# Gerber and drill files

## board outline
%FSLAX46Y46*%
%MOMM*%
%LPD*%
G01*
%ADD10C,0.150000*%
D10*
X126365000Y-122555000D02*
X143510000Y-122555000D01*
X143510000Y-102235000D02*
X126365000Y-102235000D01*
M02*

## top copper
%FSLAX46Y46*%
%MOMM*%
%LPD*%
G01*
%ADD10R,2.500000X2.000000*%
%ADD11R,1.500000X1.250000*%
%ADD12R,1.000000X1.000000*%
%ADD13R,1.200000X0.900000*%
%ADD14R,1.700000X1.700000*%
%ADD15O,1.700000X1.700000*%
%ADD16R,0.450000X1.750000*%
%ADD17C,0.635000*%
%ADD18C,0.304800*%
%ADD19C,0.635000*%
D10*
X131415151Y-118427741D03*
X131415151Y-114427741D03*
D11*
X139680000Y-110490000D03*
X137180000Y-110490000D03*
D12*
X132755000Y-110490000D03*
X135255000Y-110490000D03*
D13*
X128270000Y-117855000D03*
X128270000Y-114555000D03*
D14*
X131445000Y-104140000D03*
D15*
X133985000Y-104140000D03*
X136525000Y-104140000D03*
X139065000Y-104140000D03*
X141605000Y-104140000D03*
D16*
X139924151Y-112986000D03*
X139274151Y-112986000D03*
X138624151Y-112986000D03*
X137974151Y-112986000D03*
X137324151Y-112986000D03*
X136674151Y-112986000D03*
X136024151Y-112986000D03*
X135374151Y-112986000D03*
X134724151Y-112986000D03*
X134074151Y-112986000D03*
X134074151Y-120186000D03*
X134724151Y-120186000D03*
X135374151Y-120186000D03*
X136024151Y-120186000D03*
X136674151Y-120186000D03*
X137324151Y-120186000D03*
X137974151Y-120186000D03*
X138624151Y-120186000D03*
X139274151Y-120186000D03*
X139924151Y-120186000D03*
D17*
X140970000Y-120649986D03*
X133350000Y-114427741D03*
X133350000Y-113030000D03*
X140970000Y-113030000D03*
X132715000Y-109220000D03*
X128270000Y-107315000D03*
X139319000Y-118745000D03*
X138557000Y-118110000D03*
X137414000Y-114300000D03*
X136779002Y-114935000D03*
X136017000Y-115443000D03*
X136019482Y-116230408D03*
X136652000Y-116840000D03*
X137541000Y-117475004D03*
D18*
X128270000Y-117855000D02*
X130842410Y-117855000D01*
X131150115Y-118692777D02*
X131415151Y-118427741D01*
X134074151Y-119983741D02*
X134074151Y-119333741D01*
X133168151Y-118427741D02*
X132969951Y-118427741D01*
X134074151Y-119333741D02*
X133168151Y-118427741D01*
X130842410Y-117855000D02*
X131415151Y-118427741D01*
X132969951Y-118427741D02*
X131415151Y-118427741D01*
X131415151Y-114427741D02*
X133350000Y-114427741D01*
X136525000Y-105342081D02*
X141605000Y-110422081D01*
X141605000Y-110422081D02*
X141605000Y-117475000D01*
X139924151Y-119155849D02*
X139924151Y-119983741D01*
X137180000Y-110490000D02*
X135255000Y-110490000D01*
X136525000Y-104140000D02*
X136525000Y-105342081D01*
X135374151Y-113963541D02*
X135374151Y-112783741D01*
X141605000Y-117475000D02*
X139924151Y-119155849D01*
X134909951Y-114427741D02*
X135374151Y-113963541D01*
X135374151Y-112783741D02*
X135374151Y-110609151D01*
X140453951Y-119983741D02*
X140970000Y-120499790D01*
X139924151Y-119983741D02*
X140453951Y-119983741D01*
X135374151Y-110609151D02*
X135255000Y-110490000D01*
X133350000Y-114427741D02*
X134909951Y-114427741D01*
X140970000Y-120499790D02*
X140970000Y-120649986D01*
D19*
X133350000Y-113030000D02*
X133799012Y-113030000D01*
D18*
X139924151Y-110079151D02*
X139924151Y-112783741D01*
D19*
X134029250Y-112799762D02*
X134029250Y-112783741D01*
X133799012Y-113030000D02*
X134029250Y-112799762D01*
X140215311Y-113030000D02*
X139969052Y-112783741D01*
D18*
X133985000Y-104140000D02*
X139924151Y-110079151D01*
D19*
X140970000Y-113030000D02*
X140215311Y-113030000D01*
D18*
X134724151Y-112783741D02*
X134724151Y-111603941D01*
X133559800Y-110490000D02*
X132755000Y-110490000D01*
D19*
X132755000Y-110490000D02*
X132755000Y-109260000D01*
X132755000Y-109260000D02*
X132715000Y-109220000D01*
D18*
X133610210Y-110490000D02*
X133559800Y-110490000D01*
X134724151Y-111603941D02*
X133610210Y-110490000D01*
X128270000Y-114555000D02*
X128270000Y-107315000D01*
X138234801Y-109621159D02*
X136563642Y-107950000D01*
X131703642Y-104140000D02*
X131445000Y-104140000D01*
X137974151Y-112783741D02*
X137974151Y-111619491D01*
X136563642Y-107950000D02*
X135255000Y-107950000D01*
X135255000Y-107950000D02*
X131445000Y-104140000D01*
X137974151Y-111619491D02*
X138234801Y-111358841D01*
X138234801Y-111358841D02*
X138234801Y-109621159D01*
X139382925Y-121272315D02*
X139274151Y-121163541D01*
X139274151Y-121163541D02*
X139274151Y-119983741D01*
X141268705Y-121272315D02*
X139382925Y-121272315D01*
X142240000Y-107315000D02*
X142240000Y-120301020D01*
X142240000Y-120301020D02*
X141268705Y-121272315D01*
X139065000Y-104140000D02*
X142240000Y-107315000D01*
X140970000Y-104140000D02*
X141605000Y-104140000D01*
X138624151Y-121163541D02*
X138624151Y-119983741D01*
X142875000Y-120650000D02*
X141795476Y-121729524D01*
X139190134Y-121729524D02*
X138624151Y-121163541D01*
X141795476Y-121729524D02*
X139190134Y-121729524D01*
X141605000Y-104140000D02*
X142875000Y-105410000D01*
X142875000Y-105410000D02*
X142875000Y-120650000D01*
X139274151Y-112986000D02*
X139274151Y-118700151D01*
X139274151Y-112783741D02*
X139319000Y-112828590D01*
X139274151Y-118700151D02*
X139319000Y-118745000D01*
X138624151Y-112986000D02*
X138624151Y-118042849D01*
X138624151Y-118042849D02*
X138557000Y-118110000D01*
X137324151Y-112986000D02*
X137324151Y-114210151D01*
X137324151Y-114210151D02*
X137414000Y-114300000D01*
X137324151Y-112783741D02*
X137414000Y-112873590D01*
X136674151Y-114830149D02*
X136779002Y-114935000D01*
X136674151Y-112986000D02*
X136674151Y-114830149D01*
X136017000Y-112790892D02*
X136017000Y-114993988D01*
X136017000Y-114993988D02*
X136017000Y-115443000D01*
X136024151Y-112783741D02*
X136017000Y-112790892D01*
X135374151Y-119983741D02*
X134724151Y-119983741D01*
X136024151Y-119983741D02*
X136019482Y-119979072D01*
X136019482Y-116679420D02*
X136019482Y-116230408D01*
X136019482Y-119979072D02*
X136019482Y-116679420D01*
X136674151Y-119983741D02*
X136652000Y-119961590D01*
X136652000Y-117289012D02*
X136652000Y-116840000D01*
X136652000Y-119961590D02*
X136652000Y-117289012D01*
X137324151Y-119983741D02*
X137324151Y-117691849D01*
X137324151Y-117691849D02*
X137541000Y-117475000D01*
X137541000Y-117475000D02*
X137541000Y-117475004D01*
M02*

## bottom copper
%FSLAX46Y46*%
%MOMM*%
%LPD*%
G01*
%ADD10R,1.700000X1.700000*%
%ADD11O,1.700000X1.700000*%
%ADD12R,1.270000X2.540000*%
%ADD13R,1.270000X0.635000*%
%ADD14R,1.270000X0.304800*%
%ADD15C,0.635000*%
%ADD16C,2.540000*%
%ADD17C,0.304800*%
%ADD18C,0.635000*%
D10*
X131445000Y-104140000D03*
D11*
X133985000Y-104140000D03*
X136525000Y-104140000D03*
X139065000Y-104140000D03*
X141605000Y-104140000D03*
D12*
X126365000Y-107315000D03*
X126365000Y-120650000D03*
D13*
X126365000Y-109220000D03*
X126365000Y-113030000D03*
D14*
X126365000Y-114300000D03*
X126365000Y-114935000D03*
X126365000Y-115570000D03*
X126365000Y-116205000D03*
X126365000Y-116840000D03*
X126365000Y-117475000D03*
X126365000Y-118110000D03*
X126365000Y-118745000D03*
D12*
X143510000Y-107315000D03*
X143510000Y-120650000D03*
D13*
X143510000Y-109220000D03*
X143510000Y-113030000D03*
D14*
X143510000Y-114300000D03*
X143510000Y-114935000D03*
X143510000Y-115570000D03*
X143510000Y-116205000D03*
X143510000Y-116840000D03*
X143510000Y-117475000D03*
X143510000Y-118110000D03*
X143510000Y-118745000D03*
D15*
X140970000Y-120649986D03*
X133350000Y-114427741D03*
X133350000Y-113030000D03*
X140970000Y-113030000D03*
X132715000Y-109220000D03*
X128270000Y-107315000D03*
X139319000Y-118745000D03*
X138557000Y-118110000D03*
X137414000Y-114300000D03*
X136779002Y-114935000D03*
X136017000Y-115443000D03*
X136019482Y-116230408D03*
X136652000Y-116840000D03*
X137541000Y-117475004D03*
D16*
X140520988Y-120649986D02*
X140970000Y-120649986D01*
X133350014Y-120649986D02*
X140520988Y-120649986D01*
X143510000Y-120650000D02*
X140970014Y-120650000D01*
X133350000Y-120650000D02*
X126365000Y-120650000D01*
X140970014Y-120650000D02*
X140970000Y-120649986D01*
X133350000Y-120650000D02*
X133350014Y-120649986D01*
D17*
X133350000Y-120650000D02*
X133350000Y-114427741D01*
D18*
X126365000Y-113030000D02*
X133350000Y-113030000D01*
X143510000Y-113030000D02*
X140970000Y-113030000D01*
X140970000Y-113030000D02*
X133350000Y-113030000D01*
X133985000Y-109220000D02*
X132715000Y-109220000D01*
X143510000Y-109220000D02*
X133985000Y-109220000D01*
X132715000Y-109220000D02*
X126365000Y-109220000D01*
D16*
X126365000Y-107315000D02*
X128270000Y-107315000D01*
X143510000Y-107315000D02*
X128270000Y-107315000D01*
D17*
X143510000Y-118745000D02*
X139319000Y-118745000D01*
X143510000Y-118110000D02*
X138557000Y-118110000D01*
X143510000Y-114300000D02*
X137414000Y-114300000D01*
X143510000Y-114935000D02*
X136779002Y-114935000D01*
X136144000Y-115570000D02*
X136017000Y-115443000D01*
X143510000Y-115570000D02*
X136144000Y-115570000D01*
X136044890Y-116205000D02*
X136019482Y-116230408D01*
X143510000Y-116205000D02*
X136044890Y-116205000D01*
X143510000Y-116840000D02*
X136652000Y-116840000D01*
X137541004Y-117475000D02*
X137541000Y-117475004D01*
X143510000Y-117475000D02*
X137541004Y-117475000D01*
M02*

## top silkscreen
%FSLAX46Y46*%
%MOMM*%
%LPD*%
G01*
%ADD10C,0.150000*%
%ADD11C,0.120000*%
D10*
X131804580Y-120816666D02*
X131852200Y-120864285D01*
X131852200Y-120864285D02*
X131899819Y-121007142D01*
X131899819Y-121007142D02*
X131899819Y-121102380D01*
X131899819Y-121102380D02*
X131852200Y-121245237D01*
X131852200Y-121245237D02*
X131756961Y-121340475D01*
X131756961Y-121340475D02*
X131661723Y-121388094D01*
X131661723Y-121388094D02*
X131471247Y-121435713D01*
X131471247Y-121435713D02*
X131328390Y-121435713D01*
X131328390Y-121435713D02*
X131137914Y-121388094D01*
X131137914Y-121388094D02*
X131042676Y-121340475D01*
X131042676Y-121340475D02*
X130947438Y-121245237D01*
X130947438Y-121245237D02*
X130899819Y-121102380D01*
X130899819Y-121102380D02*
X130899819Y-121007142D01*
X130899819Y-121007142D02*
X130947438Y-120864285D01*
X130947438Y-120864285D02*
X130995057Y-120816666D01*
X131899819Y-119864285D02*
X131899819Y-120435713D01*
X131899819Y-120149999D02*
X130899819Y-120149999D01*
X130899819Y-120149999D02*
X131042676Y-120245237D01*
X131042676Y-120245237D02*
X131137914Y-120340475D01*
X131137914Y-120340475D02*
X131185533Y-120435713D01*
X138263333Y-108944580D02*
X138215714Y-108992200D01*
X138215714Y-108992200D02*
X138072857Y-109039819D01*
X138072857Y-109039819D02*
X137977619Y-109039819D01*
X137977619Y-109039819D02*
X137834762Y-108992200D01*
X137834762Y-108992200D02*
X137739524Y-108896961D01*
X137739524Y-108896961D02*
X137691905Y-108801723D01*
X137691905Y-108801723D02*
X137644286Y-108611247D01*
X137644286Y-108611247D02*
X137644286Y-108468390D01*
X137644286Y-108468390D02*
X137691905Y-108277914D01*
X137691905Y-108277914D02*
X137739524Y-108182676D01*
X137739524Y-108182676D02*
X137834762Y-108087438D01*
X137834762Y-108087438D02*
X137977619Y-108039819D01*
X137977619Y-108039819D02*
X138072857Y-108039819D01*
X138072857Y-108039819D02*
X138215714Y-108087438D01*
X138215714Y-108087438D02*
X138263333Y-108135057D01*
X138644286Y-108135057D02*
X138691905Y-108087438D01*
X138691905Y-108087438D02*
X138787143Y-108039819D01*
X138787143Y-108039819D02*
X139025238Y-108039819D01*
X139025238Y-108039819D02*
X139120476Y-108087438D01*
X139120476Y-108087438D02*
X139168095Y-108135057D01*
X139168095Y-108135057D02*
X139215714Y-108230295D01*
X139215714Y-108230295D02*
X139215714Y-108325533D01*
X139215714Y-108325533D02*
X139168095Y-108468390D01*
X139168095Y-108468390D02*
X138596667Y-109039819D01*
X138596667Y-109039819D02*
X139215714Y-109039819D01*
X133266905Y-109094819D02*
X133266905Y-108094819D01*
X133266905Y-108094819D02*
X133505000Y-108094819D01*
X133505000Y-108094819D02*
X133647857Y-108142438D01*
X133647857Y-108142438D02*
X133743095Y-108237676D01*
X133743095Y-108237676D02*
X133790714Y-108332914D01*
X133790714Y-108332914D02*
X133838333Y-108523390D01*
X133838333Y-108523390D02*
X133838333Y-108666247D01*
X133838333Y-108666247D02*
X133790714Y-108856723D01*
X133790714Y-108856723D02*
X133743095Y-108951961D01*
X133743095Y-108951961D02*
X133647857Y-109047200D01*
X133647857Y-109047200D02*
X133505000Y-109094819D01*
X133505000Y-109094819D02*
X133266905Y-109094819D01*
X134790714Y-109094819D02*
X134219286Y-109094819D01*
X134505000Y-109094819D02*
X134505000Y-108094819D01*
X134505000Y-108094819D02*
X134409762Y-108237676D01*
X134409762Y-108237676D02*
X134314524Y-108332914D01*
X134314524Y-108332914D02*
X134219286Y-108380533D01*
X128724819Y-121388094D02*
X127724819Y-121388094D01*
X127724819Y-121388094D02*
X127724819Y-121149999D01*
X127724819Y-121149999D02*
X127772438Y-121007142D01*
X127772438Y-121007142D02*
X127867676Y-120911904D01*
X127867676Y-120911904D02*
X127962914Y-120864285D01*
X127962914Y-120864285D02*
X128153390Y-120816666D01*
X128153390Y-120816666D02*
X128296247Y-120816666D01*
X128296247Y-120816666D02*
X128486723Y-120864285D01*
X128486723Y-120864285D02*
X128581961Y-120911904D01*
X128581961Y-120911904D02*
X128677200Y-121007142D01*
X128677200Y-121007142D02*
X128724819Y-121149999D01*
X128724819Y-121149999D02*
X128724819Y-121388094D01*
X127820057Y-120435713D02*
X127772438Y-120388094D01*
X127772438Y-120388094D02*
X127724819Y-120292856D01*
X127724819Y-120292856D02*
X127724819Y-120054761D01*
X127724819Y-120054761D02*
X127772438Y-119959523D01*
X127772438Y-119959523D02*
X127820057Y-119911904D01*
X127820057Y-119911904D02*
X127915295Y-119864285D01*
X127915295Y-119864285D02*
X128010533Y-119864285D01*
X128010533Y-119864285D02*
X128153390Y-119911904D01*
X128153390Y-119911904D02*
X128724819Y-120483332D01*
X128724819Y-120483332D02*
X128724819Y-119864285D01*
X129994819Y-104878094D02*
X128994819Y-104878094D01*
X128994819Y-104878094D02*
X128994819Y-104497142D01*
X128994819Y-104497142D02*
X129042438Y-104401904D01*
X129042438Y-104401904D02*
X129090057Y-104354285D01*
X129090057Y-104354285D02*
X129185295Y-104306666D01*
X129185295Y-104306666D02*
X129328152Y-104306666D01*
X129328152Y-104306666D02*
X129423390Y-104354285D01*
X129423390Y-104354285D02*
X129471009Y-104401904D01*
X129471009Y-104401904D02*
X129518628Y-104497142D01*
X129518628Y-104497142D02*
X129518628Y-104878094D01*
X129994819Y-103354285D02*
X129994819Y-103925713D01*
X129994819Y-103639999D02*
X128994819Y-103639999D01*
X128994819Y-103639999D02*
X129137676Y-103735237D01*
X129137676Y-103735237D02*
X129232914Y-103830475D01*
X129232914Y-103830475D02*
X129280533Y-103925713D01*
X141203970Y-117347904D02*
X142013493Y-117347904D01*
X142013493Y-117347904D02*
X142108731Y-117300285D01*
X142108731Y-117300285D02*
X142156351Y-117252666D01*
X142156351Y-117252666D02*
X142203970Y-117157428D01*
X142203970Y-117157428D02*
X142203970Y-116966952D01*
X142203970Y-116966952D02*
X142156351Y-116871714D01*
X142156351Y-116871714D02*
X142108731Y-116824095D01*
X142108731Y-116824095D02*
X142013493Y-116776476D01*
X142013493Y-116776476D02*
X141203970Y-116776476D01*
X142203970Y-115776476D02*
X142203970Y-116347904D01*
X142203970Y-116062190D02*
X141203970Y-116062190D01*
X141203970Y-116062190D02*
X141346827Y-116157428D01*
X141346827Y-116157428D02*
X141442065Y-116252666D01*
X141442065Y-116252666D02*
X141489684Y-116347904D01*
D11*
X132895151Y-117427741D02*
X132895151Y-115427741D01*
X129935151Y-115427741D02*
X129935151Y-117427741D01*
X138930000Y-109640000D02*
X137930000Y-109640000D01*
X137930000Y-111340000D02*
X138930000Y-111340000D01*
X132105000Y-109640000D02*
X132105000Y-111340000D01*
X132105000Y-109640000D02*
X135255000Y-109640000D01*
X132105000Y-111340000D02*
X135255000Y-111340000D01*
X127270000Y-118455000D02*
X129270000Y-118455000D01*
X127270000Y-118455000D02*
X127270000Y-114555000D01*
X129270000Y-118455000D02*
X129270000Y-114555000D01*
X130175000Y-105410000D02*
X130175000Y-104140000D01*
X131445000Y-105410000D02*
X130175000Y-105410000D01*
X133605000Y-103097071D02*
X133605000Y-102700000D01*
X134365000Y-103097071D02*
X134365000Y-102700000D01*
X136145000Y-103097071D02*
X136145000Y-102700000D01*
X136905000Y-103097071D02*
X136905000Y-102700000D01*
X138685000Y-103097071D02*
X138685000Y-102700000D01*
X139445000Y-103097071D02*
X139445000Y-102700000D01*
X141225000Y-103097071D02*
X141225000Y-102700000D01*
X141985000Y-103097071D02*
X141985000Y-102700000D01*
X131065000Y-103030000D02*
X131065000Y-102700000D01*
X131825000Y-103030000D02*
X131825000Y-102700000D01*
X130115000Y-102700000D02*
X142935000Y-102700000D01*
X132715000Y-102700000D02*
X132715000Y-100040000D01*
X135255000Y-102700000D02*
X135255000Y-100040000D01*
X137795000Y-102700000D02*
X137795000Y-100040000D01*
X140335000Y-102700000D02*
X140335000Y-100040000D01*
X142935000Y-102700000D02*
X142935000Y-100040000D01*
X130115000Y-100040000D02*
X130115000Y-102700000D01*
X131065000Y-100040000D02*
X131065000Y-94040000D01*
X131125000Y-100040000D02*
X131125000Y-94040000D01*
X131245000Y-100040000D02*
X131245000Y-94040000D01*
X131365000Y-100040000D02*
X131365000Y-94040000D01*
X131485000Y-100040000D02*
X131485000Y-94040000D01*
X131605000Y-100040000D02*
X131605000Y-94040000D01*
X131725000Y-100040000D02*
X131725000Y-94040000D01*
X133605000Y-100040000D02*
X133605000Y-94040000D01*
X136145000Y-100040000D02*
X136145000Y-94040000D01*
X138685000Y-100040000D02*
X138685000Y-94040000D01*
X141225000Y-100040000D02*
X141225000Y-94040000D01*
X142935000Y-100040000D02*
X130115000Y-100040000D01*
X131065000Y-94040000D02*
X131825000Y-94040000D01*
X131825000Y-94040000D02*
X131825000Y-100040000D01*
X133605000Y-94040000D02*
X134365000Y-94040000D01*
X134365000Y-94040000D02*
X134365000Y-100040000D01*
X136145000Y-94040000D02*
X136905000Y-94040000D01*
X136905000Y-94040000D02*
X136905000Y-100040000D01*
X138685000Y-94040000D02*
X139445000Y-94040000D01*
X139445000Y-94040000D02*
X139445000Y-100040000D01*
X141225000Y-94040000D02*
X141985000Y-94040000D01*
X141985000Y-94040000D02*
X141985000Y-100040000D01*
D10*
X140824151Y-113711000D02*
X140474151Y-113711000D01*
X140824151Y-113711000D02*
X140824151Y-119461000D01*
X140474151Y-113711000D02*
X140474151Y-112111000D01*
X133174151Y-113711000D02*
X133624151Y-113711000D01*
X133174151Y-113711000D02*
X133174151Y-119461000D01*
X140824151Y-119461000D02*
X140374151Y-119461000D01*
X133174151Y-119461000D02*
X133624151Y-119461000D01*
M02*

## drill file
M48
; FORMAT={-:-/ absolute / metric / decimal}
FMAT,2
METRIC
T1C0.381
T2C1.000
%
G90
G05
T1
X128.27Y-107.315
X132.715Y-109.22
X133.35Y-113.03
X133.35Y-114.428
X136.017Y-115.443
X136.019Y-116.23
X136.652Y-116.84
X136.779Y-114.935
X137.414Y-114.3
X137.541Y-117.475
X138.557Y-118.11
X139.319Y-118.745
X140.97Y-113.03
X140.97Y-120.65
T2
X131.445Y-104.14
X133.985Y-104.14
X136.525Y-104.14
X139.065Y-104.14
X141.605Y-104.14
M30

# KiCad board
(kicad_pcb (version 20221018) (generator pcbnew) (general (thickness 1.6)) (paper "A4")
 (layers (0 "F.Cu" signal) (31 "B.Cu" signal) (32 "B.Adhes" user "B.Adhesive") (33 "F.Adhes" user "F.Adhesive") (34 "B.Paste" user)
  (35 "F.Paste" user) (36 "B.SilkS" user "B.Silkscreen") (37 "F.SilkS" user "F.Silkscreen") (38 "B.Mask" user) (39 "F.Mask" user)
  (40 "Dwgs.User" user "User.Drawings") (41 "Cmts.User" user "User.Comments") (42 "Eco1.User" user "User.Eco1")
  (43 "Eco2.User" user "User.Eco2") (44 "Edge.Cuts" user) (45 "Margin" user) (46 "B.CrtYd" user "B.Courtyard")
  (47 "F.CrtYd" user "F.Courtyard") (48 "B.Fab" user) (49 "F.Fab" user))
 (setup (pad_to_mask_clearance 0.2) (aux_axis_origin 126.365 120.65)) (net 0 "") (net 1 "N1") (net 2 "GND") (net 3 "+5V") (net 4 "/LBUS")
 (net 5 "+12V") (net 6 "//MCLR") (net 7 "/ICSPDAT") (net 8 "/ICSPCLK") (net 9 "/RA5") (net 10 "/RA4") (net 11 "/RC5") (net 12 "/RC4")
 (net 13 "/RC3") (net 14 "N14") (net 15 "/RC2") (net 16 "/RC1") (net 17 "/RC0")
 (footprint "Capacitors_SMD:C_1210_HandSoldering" (layer "F.Cu") (at 131.415151 116.427741 90)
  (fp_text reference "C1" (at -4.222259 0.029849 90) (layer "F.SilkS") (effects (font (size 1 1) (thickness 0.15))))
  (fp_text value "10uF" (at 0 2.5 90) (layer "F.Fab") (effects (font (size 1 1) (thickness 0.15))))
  (fp_line (start -1 1.48) (end 1 1.48) (stroke (width 0.12) (type solid)) (layer "F.SilkS"))
  (fp_line (start 1 -1.48) (end -1 -1.48) (stroke (width 0.12) (type solid)) (layer "F.SilkS"))
  (pad "1" smd rect (at -2 0 90) (size 2 2.5) (layers "F.Cu" "F.Paste" "F.Mask") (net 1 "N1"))
  (pad "2" smd rect (at 2 0 90) (size 2 2.5) (layers "F.Cu" "F.Paste" "F.Mask") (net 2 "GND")))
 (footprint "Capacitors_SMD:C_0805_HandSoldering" (layer "F.Cu") (at 138.43 110.49 180)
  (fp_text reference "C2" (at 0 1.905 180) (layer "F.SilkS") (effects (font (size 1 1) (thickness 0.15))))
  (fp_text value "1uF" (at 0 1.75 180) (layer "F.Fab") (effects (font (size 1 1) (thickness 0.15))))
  (fp_line (start -0.5 0.85) (end 0.5 0.85) (stroke (width 0.12) (type solid)) (layer "F.SilkS"))
  (fp_line (start 0.5 -0.85) (end -0.5 -0.85) (stroke (width 0.12) (type solid)) (layer "F.SilkS"))
  (pad "1" smd rect (at -1.25 0 180) (size 1.5 1.25) (layers "F.Cu" "F.Paste" "F.Mask") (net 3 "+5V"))
  (pad "2" smd rect (at 1.25 0 180) (size 1.5 1.25) (layers "F.Cu" "F.Paste" "F.Mask") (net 2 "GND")))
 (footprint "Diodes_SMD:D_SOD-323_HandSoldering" (layer "F.Cu") (at 134.005 110.49)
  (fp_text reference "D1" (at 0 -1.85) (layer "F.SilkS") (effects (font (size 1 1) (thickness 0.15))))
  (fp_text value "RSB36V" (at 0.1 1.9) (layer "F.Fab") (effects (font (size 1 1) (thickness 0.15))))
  (fp_line (start -1.9 -0.85) (end -1.9 0.85) (stroke (width 0.12) (type solid)) (layer "F.SilkS"))
  (fp_line (start -1.9 -0.85) (end 1.25 -0.85) (stroke (width 0.12) (type solid)) (layer "F.SilkS"))
  (fp_line (start -1.9 0.85) (end 1.25 0.85) (stroke (width 0.12) (type solid)) (layer "F.SilkS"))
  (pad "1" smd rect (at -1.25 0) (size 1 1) (layers "F.Cu" "F.Paste" "F.Mask") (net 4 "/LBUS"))
  (pad "2" smd rect (at 1.25 0) (size 1 1) (layers "F.Cu" "F.Paste" "F.Mask") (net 2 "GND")))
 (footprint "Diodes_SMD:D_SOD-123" (layer "F.Cu") (at 128.27 116.205 90)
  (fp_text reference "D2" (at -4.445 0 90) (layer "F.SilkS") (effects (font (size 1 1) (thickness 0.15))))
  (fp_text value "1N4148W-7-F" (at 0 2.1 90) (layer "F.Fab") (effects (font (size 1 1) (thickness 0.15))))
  (fp_line (start -2.25 -1) (end -2.25 1) (stroke (width 0.12) (type solid)) (layer "F.SilkS"))
  (fp_line (start -2.25 -1) (end 1.65 -1) (stroke (width 0.12) (type solid)) (layer "F.SilkS"))
  (fp_line (start -2.25 1) (end 1.65 1) (stroke (width 0.12) (type solid)) (layer "F.SilkS"))
  (pad "1" smd rect (at -1.65 0 90) (size 0.9 1.2) (layers "F.Cu" "F.Paste" "F.Mask") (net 1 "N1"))
  (pad "2" smd rect (at 1.65 0 90) (size 0.9 1.2) (layers "F.Cu" "F.Paste" "F.Mask") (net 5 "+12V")))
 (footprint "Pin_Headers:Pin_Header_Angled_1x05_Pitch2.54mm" (layer "F.Cu") (at 131.445 104.14 90)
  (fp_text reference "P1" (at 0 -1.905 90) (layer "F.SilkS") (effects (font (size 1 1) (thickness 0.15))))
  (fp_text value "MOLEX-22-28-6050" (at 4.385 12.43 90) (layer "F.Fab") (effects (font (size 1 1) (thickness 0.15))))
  (fp_line (start -1.27 -1.27) (end 0 -1.27) (stroke (width 0.12) (type solid)) (layer "F.SilkS"))
  (fp_line (start -1.27 0) (end -1.27 -1.27) (stroke (width 0.12) (type solid)) (layer "F.SilkS"))
  (fp_line (start 1.042929 2.16) (end 1.44 2.16) (stroke (width 0.12) (type solid)) (layer "F.SilkS"))
  (fp_line (start 1.042929 2.92) (end 1.44 2.92) (stroke (width 0.12) (type solid)) (layer "F.SilkS"))
  (fp_line (start 1.042929 4.7) (end 1.44 4.7) (stroke (width 0.12) (type solid)) (layer "F.SilkS"))
  (fp_line (start 1.042929 5.46) (end 1.44 5.46) (stroke (width 0.12) (type solid)) (layer "F.SilkS"))
  (fp_line (start 1.042929 7.24) (end 1.44 7.24) (stroke (width 0.12) (type solid)) (layer "F.SilkS"))
  (fp_line (start 1.042929 8) (end 1.44 8) (stroke (width 0.12) (type solid)) (layer "F.SilkS"))
  (fp_line (start 1.042929 9.78) (end 1.44 9.78) (stroke (width 0.12) (type solid)) (layer "F.SilkS"))
  (fp_line (start 1.042929 10.54) (end 1.44 10.54) (stroke (width 0.12) (type solid)) (layer "F.SilkS"))
  (fp_line (start 1.11 -0.38) (end 1.44 -0.38) (stroke (width 0.12) (type solid)) (layer "F.SilkS"))
  (fp_line (start 1.11 0.38) (end 1.44 0.38) (stroke (width 0.12) (type solid)) (layer "F.SilkS"))
  (fp_line (start 1.44 -1.33) (end 1.44 11.49) (stroke (width 0.12) (type solid)) (layer "F.SilkS"))
  (fp_line (start 1.44 1.27) (end 4.1 1.27) (stroke (width 0.12) (type solid)) (layer "F.SilkS"))
  (fp_line (start 1.44 3.81) (end 4.1 3.81) (stroke (width 0.12) (type solid)) (layer "F.SilkS"))
  (fp_line (start 1.44 6.35) (end 4.1 6.35) (stroke (width 0.12) (type solid)) (layer "F.SilkS"))
  (fp_line (start 1.44 8.89) (end 4.1 8.89) (stroke (width 0.12) (type solid)) (layer "F.SilkS"))
  (fp_line (start 1.44 11.49) (end 4.1 11.49) (stroke (width 0.12) (type solid)) (layer "F.SilkS"))
  (fp_line (start 4.1 -1.33) (end 1.44 -1.33) (stroke (width 0.12) (type solid)) (layer "F.SilkS"))
  (fp_line (start 4.1 -0.38) (end 10.1 -0.38) (stroke (width 0.12) (type solid)) (layer "F.SilkS"))
  (fp_line (start 4.1 -0.32) (end 10.1 -0.32) (stroke (width 0.12) (type solid)) (layer "F.SilkS"))
  (fp_line (start 4.1 -0.2) (end 10.1 -0.2) (stroke (width 0.12) (type solid)) (layer "F.SilkS"))
  (fp_line (start 4.1 -0.08) (end 10.1 -0.08) (stroke (width 0.12) (type solid)) (layer "F.SilkS"))
  (fp_line (start 4.1 0.04) (end 10.1 0.04) (stroke (width 0.12) (type solid)) (layer "F.SilkS"))
  (fp_line (start 4.1 0.16) (end 10.1 0.16) (stroke (width 0.12) (type solid)) (layer "F.SilkS"))
  (fp_line (start 4.1 0.28) (end 10.1 0.28) (stroke (width 0.12) (type solid)) (layer "F.SilkS"))
  (fp_line (start 4.1 2.16) (end 10.1 2.16) (stroke (width 0.12) (type solid)) (layer "F.SilkS"))
  (fp_line (start 4.1 4.7) (end 10.1 4.7) (stroke (width 0.12) (type solid)) (layer "F.SilkS"))
  (fp_line (start 4.1 7.24) (end 10.1 7.24) (stroke (width 0.12) (type solid)) (layer "F.SilkS"))
  (fp_line (start 4.1 9.78) (end 10.1 9.78) (stroke (width 0.12) (type solid)) (layer "F.SilkS"))
  (fp_line (start 4.1 11.49) (end 4.1 -1.33) (stroke (width 0.12) (type solid)) (layer "F.SilkS"))
  (fp_line (start 10.1 -0.38) (end 10.1 0.38) (stroke (width 0.12) (type solid)) (layer "F.SilkS"))
  (fp_line (start 10.1 0.38) (end 4.1 0.38) (stroke (width 0.12) (type solid)) (layer "F.SilkS"))
  (fp_line (start 10.1 2.16) (end 10.1 2.92) (stroke (width 0.12) (type solid)) (layer "F.SilkS"))
  (fp_line (start 10.1 2.92) (end 4.1 2.92) (stroke (width 0.12) (type solid)) (layer "F.SilkS"))
  (fp_line (start 10.1 4.7) (end 10.1 5.46) (stroke (width 0.12) (type solid)) (layer "F.SilkS"))
  (fp_line (start 10.1 5.46) (end 4.1 5.46) (stroke (width 0.12) (type solid)) (layer "F.SilkS"))
  (fp_line (start 10.1 7.24) (end 10.1 8) (stroke (width 0.12) (type solid)) (layer "F.SilkS"))
  (fp_line (start 10.1 8) (end 4.1 8) (stroke (width 0.12) (type solid)) (layer "F.SilkS"))
  (fp_line (start 10.1 9.78) (end 10.1 10.54) (stroke (width 0.12) (type solid)) (layer "F.SilkS"))
  (fp_line (start 10.1 10.54) (end 4.1 10.54) (stroke (width 0.12) (type solid)) (layer "F.SilkS"))
  (pad "1" thru_hole rect (at 0 0 90) (size 1.7 1.7) (drill 1) (layers "*.Cu" "*.Mask") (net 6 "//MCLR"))
  (pad "2" thru_hole oval (at 0 2.54 90) (size 1.7 1.7) (drill 1) (layers "*.Cu" "*.Mask") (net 3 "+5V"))
  (pad "3" thru_hole oval (at 0 5.08 90) (size 1.7 1.7) (drill 1) (layers "*.Cu" "*.Mask") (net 2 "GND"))
  (pad "4" thru_hole oval (at 0 7.62 90) (size 1.7 1.7) (drill 1) (layers "*.Cu" "*.Mask") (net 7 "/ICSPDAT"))
  (pad "5" thru_hole oval (at 0 10.16 90) (size 1.7 1.7) (drill 1) (layers "*.Cu" "*.Mask") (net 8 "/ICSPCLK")))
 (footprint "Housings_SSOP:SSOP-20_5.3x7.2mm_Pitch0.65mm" (layer "F.Cu") (at 136.999151 116.586 -90)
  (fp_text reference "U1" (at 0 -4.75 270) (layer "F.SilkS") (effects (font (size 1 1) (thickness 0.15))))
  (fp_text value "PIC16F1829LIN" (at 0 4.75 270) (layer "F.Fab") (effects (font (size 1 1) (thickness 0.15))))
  (fp_line (start -2.875 -3.825) (end -2.875 -3.475) (stroke (width 0.15) (type solid)) (layer "F.SilkS"))
  (fp_line (start -2.875 -3.825) (end 2.875 -3.825) (stroke (width 0.15) (type solid)) (layer "F.SilkS"))
  (fp_line (start -2.875 -3.475) (end -4.475 -3.475) (stroke (width 0.15) (type solid)) (layer "F.SilkS"))
  (fp_line (start -2.875 3.825) (end -2.875 3.375) (stroke (width 0.15) (type solid)) (layer "F.SilkS"))
  (fp_line (start -2.875 3.825) (end 2.875 3.825) (stroke (width 0.15) (type solid)) (layer "F.SilkS"))
  (fp_line (start 2.875 -3.825) (end 2.875 -3.375) (stroke (width 0.15) (type solid)) (layer "F.SilkS"))
  (fp_line (start 2.875 3.825) (end 2.875 3.375) (stroke (width 0.15) (type solid)) (layer "F.SilkS"))
  (pad "1" smd rect (at -3.6 -2.925 270) (size 1.75 0.45) (layers "F.Cu" "F.Paste" "F.Mask") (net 3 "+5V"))
  (pad "2" smd rect (at -3.6 -2.275 270) (size 1.75 0.45) (layers "F.Cu" "F.Paste" "F.Mask") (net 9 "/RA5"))
  (pad "3" smd rect (at -3.6 -1.625 270) (size 1.75 0.45) (layers "F.Cu" "F.Paste" "F.Mask") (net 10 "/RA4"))
  (pad "4" smd rect (at -3.6 -0.975 270) (size 1.75 0.45) (layers "F.Cu" "F.Paste" "F.Mask") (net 6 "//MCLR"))
  (pad "5" smd rect (at -3.6 -0.325 270) (size 1.75 0.45) (layers "F.Cu" "F.Paste" "F.Mask") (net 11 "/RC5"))
  (pad "6" smd rect (at -3.6 0.325 270) (size 1.75 0.45) (layers "F.Cu" "F.Paste" "F.Mask") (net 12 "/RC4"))
  (pad "7" smd rect (at -3.6 0.975 270) (size 1.75 0.45) (layers "F.Cu" "F.Paste" "F.Mask") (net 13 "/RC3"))
  (pad "8" smd rect (at -3.6 1.625 270) (size 1.75 0.45) (layers "F.Cu" "F.Paste" "F.Mask") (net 2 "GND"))
  (pad "9" smd rect (at -3.6 2.275 270) (size 1.75 0.45) (layers "F.Cu" "F.Paste" "F.Mask") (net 4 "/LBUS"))
  (pad "10" smd rect (at -3.6 2.925 270) (size 1.75 0.45) (layers "F.Cu" "F.Paste" "F.Mask") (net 3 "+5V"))
  (pad "11" smd rect (at 3.6 2.925 270) (size 1.75 0.45) (layers "F.Cu" "F.Paste" "F.Mask") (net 1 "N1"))
  (pad "12" smd rect (at 3.6 2.275 270) (size 1.75 0.45) (layers "F.Cu" "F.Paste" "F.Mask") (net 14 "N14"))
  (pad "13" smd rect (at 3.6 1.625 270) (size 1.75 0.45) (layers "F.Cu" "F.Paste" "F.Mask") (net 14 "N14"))
  (pad "14" smd rect (at 3.6 0.975 270) (size 1.75 0.45) (layers "F.Cu" "F.Paste" "F.Mask") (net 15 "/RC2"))
  (pad "15" smd rect (at 3.6 0.325 270) (size 1.75 0.45) (layers "F.Cu" "F.Paste" "F.Mask") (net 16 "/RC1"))
  (pad "16" smd rect (at 3.6 -0.325 270) (size 1.75 0.45) (layers "F.Cu" "F.Paste" "F.Mask") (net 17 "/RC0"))
  (pad "17" smd rect (at 3.6 -0.975 270) (size 1.75 0.45) (layers "F.Cu" "F.Paste" "F.Mask"))
  (pad "18" smd rect (at 3.6 -1.625 270) (size 1.75 0.45) (layers "F.Cu" "F.Paste" "F.Mask") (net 8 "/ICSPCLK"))
  (pad "19" smd rect (at 3.6 -2.275 270) (size 1.75 0.45) (layers "F.Cu" "F.Paste" "F.Mask") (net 7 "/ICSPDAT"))
  (pad "20" smd rect (at 3.6 -2.925 270) (size 1.75 0.45) (layers "F.Cu" "F.Paste" "F.Mask") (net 2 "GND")))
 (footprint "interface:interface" (layer "F.Cu") (at 126.365 102.87)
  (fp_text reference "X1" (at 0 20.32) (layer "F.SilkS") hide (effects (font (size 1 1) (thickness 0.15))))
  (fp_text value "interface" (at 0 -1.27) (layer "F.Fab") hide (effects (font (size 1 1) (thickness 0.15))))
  (pad "1" smd rect (at 0 4.445) (size 1.27 2.54) (layers "B.Cu") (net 5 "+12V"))
  (pad "2" smd rect (at 0 17.78) (size 1.27 2.54) (layers "B.Cu") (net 2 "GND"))
  (pad "3" smd rect (at 0 6.35) (size 1.27 0.635) (layers "B.Cu") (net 4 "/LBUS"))
  (pad "4" smd rect (at 0 10.16) (size 1.27 0.635) (layers "B.Cu") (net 3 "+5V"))
  (pad "5" smd rect (at 0 11.43) (size 1.27 0.3048) (layers "B.Cu"))
  (pad "6" smd rect (at 0 12.065) (size 1.27 0.3048) (layers "B.Cu"))
  (pad "7" smd rect (at 0 12.7) (size 1.27 0.3048) (layers "B.Cu"))
  (pad "8" smd rect (at 0 13.335) (size 1.27 0.3048) (layers "B.Cu"))
  (pad "9" smd rect (at 0 13.97) (size 1.27 0.3048) (layers "B.Cu"))
  (pad "10" smd rect (at 0 14.605) (size 1.27 0.3048) (layers "B.Cu"))
  (pad "11" smd rect (at 0 15.24) (size 1.27 0.3048) (layers "B.Cu"))
  (pad "12" smd rect (at 0 15.875) (size 1.27 0.3048) (layers "B.Cu")))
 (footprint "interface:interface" (layer "F.Cu") (at 143.51 102.87)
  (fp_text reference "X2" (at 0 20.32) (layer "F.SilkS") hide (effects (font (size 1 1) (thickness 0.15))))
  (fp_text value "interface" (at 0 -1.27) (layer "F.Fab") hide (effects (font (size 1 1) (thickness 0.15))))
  (pad "1" smd rect (at 0 4.445) (size 1.27 2.54) (layers "B.Cu") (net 5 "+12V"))
  (pad "2" smd rect (at 0 17.78) (size 1.27 2.54) (layers "B.Cu") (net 2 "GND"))
  (pad "3" smd rect (at 0 6.35) (size 1.27 0.635) (layers "B.Cu") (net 4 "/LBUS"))
  (pad "4" smd rect (at 0 10.16) (size 1.27 0.635) (layers "B.Cu") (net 3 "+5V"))
  (pad "5" smd rect (at 0 11.43) (size 1.27 0.3048) (layers "B.Cu") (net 11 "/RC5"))
  (pad "6" smd rect (at 0 12.065) (size 1.27 0.3048) (layers "B.Cu") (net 12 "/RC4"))
  (pad "7" smd rect (at 0 12.7) (size 1.27 0.3048) (layers "B.Cu") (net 13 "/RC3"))
  (pad "8" smd rect (at 0 13.335) (size 1.27 0.3048) (layers "B.Cu") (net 15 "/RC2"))
  (pad "9" smd rect (at 0 13.97) (size 1.27 0.3048) (layers "B.Cu") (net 16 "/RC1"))
  (pad "10" smd rect (at 0 14.605) (size 1.27 0.3048) (layers "B.Cu") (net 17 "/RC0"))
  (pad "11" smd rect (at 0 15.24) (size 1.27 0.3048) (layers "B.Cu") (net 10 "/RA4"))
  (pad "12" smd rect (at 0 15.875) (size 1.27 0.3048) (layers "B.Cu") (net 9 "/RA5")))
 (gr_line (start 126.365 122.555) (end 143.51 122.555) (stroke (width 0.15) (type solid)) (layer "Edge.Cuts"))
 (gr_line (start 143.51 102.235) (end 126.365 102.235) (stroke (width 0.15) (type solid)) (layer "Edge.Cuts"))
 (segment (start 128.27 117.855) (end 130.84241 117.855) (width 0.3048) (layer "F.Cu") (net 1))
 (segment (start 131.150115 118.692777) (end 131.415151 118.427741) (width 0.3048) (layer "F.Cu") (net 1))
 (segment (start 134.074151 119.983741) (end 134.074151 119.333741) (width 0.3048) (layer "F.Cu") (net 1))
 (segment (start 133.168151 118.427741) (end 132.969951 118.427741) (width 0.3048) (layer "F.Cu") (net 1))
 (segment (start 134.074151 119.333741) (end 133.168151 118.427741) (width 0.3048) (layer "F.Cu") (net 1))
 (segment (start 130.84241 117.855) (end 131.415151 118.427741) (width 0.3048) (layer "F.Cu") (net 1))
 (segment (start 132.969951 118.427741) (end 131.415151 118.427741) (width 0.3048) (layer "F.Cu") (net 1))
 (segment (start 131.415151 114.427741) (end 133.35 114.427741) (width 0.3048) (layer "F.Cu") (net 2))
 (segment (start 136.525 105.342081) (end 141.605 110.422081) (width 0.3048) (layer "F.Cu") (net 2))
 (segment (start 141.605 110.422081) (end 141.605 117.475) (width 0.3048) (layer "F.Cu") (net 2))
 (segment (start 139.924151 119.155849) (end 139.924151 119.983741) (width 0.3048) (layer "F.Cu") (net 2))
 (segment (start 137.18 110.49) (end 135.255 110.49) (width 0.3048) (layer "F.Cu") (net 2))
 (segment (start 136.525 104.14) (end 136.525 105.342081) (width 0.3048) (layer "F.Cu") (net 2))
 (segment (start 135.374151 113.963541) (end 135.374151 112.783741) (width 0.3048) (layer "F.Cu") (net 2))
 (segment (start 141.605 117.475) (end 139.924151 119.155849) (width 0.3048) (layer "F.Cu") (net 2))
 (segment (start 134.909951 114.427741) (end 135.374151 113.963541) (width 0.3048) (layer "F.Cu") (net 2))
 (segment (start 135.374151 112.783741) (end 135.374151 110.609151) (width 0.3048) (layer "F.Cu") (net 2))
 (segment (start 140.453951 119.983741) (end 140.97 120.49979) (width 0.3048) (layer "F.Cu") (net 2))
 (segment (start 139.924151 119.983741) (end 140.453951 119.983741) (width 0.3048) (layer "F.Cu") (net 2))
 (segment (start 135.374151 110.609151) (end 135.255 110.49) (width 0.3048) (layer "F.Cu") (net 2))
 (segment (start 133.35 114.427741) (end 134.909951 114.427741) (width 0.3048) (layer "F.Cu") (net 2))
 (segment (start 140.97 120.49979) (end 140.97 120.649986) (width 0.3048) (layer "F.Cu") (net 2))
 (via (at 140.97 120.649986) (size 0.635) (drill 0.381) (layers "F.Cu" "B.Cu") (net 2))
 (via (at 133.35 114.427741) (size 0.635) (drill 0.381) (layers "F.Cu" "B.Cu") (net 2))
 (segment (start 140.520988 120.649986) (end 140.97 120.649986) (width 2.54) (layer "B.Cu") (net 2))
 (segment (start 133.350014 120.649986) (end 140.520988 120.649986) (width 2.54) (layer "B.Cu") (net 2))
 (segment (start 143.51 120.65) (end 140.970014 120.65) (width 2.54) (layer "B.Cu") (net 2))
 (segment (start 133.35 120.65) (end 126.365 120.65) (width 2.54) (layer "B.Cu") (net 2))
 (segment (start 140.970014 120.65) (end 140.97 120.649986) (width 2.54) (layer "B.Cu") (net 2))
 (segment (start 133.35 120.65) (end 133.350014 120.649986) (width 2.54) (layer "B.Cu") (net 2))
 (segment (start 133.35 120.65) (end 133.35 114.427741) (width 0.3048) (layer "B.Cu") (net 2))
 (segment (start 133.35 113.03) (end 133.799012 113.03) (width 0.635) (layer "F.Cu") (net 3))
 (segment (start 139.924151 110.079151) (end 139.924151 112.783741) (width 0.3048) (layer "F.Cu") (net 3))
 (segment (start 134.02925 112.799762) (end 134.02925 112.783741) (width 0.635) (layer "F.Cu") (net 3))
 (segment (start 133.799012 113.03) (end 134.02925 112.799762) (width 0.635) (layer "F.Cu") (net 3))
 (segment (start 140.215311 113.03) (end 139.969052 112.783741) (width 0.635) (layer "F.Cu") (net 3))
 (segment (start 133.985 104.14) (end 139.924151 110.079151) (width 0.3048) (layer "F.Cu") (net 3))
 (segment (start 140.97 113.03) (end 140.215311 113.03) (width 0.635) (layer "F.Cu") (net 3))
 (via (at 133.35 113.03) (size 0.635) (drill 0.381) (layers "F.Cu" "B.Cu") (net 3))
 (via (at 140.97 113.03) (size 0.635) (drill 0.381) (layers "F.Cu" "B.Cu") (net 3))
 (segment (start 126.365 113.03) (end 133.35 113.03) (width 0.635) (layer "B.Cu") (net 3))
 (segment (start 143.51 113.03) (end 140.97 113.03) (width 0.635) (layer "B.Cu") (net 3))
 (segment (start 140.97 113.03) (end 133.35 113.03) (width 0.635) (layer "B.Cu") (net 3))
 (segment (start 134.724151 112.783741) (end 134.724151 111.603941) (width 0.3048) (layer "F.Cu") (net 4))
 (segment (start 133.5598 110.49) (end 132.755 110.49) (width 0.3048) (layer "F.Cu") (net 4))
 (segment (start 132.755 110.49) (end 132.755 109.26) (width 0.635) (layer "F.Cu") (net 4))
 (segment (start 132.755 109.26) (end 132.715 109.22) (width 0.635) (layer "F.Cu") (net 4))
 (segment (start 133.61021 110.49) (end 133.5598 110.49) (width 0.3048) (layer "F.Cu") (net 4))
 (segment (start 134.724151 111.603941) (end 133.61021 110.49) (width 0.3048) (layer "F.Cu") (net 4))
 (via (at 132.715 109.22) (size 0.635) (drill 0.381) (layers "F.Cu" "B.Cu") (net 4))
 (segment (start 133.985 109.22) (end 132.715 109.22) (width 0.635) (layer "B.Cu") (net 4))
 (segment (start 143.51 109.22) (end 133.985 109.22) (width 0.635) (layer "B.Cu") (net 4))
 (segment (start 132.715 109.22) (end 126.365 109.22) (width 0.635) (layer "B.Cu") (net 4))
 (segment (start 128.27 114.555) (end 128.27 107.315) (width 0.3048) (layer "F.Cu") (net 5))
 (via (at 128.27 107.315) (size 0.635) (drill 0.381) (layers "F.Cu" "B.Cu") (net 5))
 (segment (start 126.365 107.315) (end 128.27 107.315) (width 2.54) (layer "B.Cu") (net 5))
 (segment (start 143.51 107.315) (end 128.27 107.315) (width 2.54) (layer "B.Cu") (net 5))
 (segment (start 138.234801 109.621159) (end 136.563642 107.95) (width 0.3048) (layer "F.Cu") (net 6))
 (segment (start 131.703642 104.14) (end 131.445 104.14) (width 0.3048) (layer "F.Cu") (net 6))
 (segment (start 137.974151 112.783741) (end 137.974151 111.619491) (width 0.3048) (layer "F.Cu") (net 6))
 (segment (start 136.563642 107.95) (end 135.255 107.95) (width 0.3048) (layer "F.Cu") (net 6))
 (segment (start 135.255 107.95) (end 131.445 104.14) (width 0.3048) (layer "F.Cu") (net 6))
 (segment (start 137.974151 111.619491) (end 138.234801 111.358841) (width 0.3048) (layer "F.Cu") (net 6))
 (segment (start 138.234801 111.358841) (end 138.234801 109.621159) (width 0.3048) (layer "F.Cu") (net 6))
 (segment (start 139.382925 121.272315) (end 139.274151 121.163541) (width 0.3048) (layer "F.Cu") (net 7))
 (segment (start 139.274151 121.163541) (end 139.274151 119.983741) (width 0.3048) (layer "F.Cu") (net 7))
 (segment (start 141.268705 121.272315) (end 139.382925 121.272315) (width 0.3048) (layer "F.Cu") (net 7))
 (segment (start 142.24 107.315) (end 142.24 120.30102) (width 0.3048) (layer "F.Cu") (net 7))
 (segment (start 142.24 120.30102) (end 141.268705 121.272315) (width 0.3048) (layer "F.Cu") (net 7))
 (segment (start 139.065 104.14) (end 142.24 107.315) (width 0.3048) (layer "F.Cu") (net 7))
 (segment (start 140.97 104.14) (end 141.605 104.14) (width 0.3048) (layer "F.Cu") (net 8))
 (segment (start 138.624151 121.163541) (end 138.624151 119.983741) (width 0.3048) (layer "F.Cu") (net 8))
 (segment (start 142.875 120.65) (end 141.795476 121.729524) (width 0.3048) (layer "F.Cu") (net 8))
 (segment (start 139.190134 121.729524) (end 138.624151 121.163541) (width 0.3048) (layer "F.Cu") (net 8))
 (segment (start 141.795476 121.729524) (end 139.190134 121.729524) (width 0.3048) (layer "F.Cu") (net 8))
 (segment (start 141.605 104.14) (end 142.875 105.41) (width 0.3048) (layer "F.Cu") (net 8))
 (segment (start 142.875 105.41) (end 142.875 120.65) (width 0.3048) (layer "F.Cu") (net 8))
 (segment (start 139.274151 112.986) (end 139.274151 118.700151) (width 0.3048) (layer "F.Cu") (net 9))
 (segment (start 139.274151 112.783741) (end 139.319 112.82859) (width 0.3048) (layer "F.Cu") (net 9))
 (segment (start 139.274151 118.700151) (end 139.319 118.745) (width 0.3048) (layer "F.Cu") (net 9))
 (via (at 139.319 118.745) (size 0.635) (drill 0.381) (layers "F.Cu" "B.Cu") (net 9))
 (segment (start 143.51 118.745) (end 139.319 118.745) (width 0.3048) (layer "B.Cu") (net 9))
 (segment (start 138.624151 112.986) (end 138.624151 118.042849) (width 0.3048) (layer "F.Cu") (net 10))
 (segment (start 138.624151 118.042849) (end 138.557 118.11) (width 0.3048) (layer "F.Cu") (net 10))
 (via (at 138.557 118.11) (size 0.635) (drill 0.381) (layers "F.Cu" "B.Cu") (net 10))
 (segment (start 143.51 118.11) (end 138.557 118.11) (width 0.3048) (layer "B.Cu") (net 10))
 (segment (start 137.324151 112.986) (end 137.324151 114.210151) (width 0.3048) (layer "F.Cu") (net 11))
 (segment (start 137.324151 114.210151) (end 137.414 114.3) (width 0.3048) (layer "F.Cu") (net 11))
 (segment (start 137.324151 112.783741) (end 137.414 112.87359) (width 0.3048) (layer "F.Cu") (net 11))
 (via (at 137.414 114.3) (size 0.635) (drill 0.381) (layers "F.Cu" "B.Cu") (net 11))
 (segment (start 143.51 114.3) (end 137.414 114.3) (width 0.3048) (layer "B.Cu") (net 11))
 (segment (start 136.674151 114.830149) (end 136.779002 114.935) (width 0.3048) (layer "F.Cu") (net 12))
 (segment (start 136.674151 112.986) (end 136.674151 114.830149) (width 0.3048) (layer "F.Cu") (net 12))
 (via (at 136.779002 114.935) (size 0.635) (drill 0.381) (layers "F.Cu" "B.Cu") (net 12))
 (segment (start 143.51 114.935) (end 136.779002 114.935) (width 0.3048) (layer "B.Cu") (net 12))
 (segment (start 136.017 112.790892) (end 136.017 114.993988) (width 0.3048) (layer "F.Cu") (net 13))
 (segment (start 136.017 114.993988) (end 136.017 115.443) (width 0.3048) (layer "F.Cu") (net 13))
 (segment (start 136.024151 112.783741) (end 136.017 112.790892) (width 0.3048) (layer "F.Cu") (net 13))
 (via (at 136.017 115.443) (size 0.635) (drill 0.381) (layers "F.Cu" "B.Cu") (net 13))
 (segment (start 136.144 115.57) (end 136.017 115.443) (width 0.3048) (layer "B.Cu") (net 13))
 (segment (start 143.51 115.57) (end 136.144 115.57) (width 0.3048) (layer "B.Cu") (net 13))
 (segment (start 135.374151 119.983741) (end 134.724151 119.983741) (width 0.3048) (layer "F.Cu") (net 14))
 (segment (start 136.024151 119.983741) (end 136.019482 119.979072) (width 0.3048) (layer "F.Cu") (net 15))
 (segment (start 136.019482 116.67942) (end 136.019482 116.230408) (width 0.3048) (layer "F.Cu") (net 15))
 (segment (start 136.019482 119.979072) (end 136.019482 116.67942) (width 0.3048) (layer "F.Cu") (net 15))
 (via (at 136.019482 116.230408) (size 0.635) (drill 0.381) (layers "F.Cu" "B.Cu") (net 15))
 (segment (start 136.04489 116.205) (end 136.019482 116.230408) (width 0.3048) (layer "B.Cu") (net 15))
 (segment (start 143.51 116.205) (end 136.04489 116.205) (width 0.3048) (layer "B.Cu") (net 15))
 (segment (start 136.674151 119.983741) (end 136.652 119.96159) (width 0.3048) (layer "F.Cu") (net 16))
 (segment (start 136.652 117.289012) (end 136.652 116.84) (width 0.3048) (layer "F.Cu") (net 16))
 (segment (start 136.652 119.96159) (end 136.652 117.289012) (width 0.3048) (layer "F.Cu") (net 16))
 (via (at 136.652 116.84) (size 0.635) (drill 0.381) (layers "F.Cu" "B.Cu") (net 16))
 (segment (start 143.51 116.84) (end 136.652 116.84) (width 0.3048) (layer "B.Cu") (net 16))
 (segment (start 137.324151 119.983741) (end 137.324151 117.691849) (width 0.3048) (layer "F.Cu") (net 17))
 (segment (start 137.324151 117.691849) (end 137.541 117.475) (width 0.3048) (layer "F.Cu") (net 17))
 (segment (start 137.541 117.475) (end 137.541 117.475004) (width 0.3048) (layer "F.Cu") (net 17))
 (via (at 137.541 117.475004) (size 0.635) (drill 0.381) (layers "F.Cu" "B.Cu") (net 17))
 (segment (start 137.541004 117.475) (end 137.541 117.475004) (width 0.3048) (layer "B.Cu") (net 17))
 (segment (start 143.51 117.475) (end 137.541004 117.475) (width 0.3048) (layer "B.Cu") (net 17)))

